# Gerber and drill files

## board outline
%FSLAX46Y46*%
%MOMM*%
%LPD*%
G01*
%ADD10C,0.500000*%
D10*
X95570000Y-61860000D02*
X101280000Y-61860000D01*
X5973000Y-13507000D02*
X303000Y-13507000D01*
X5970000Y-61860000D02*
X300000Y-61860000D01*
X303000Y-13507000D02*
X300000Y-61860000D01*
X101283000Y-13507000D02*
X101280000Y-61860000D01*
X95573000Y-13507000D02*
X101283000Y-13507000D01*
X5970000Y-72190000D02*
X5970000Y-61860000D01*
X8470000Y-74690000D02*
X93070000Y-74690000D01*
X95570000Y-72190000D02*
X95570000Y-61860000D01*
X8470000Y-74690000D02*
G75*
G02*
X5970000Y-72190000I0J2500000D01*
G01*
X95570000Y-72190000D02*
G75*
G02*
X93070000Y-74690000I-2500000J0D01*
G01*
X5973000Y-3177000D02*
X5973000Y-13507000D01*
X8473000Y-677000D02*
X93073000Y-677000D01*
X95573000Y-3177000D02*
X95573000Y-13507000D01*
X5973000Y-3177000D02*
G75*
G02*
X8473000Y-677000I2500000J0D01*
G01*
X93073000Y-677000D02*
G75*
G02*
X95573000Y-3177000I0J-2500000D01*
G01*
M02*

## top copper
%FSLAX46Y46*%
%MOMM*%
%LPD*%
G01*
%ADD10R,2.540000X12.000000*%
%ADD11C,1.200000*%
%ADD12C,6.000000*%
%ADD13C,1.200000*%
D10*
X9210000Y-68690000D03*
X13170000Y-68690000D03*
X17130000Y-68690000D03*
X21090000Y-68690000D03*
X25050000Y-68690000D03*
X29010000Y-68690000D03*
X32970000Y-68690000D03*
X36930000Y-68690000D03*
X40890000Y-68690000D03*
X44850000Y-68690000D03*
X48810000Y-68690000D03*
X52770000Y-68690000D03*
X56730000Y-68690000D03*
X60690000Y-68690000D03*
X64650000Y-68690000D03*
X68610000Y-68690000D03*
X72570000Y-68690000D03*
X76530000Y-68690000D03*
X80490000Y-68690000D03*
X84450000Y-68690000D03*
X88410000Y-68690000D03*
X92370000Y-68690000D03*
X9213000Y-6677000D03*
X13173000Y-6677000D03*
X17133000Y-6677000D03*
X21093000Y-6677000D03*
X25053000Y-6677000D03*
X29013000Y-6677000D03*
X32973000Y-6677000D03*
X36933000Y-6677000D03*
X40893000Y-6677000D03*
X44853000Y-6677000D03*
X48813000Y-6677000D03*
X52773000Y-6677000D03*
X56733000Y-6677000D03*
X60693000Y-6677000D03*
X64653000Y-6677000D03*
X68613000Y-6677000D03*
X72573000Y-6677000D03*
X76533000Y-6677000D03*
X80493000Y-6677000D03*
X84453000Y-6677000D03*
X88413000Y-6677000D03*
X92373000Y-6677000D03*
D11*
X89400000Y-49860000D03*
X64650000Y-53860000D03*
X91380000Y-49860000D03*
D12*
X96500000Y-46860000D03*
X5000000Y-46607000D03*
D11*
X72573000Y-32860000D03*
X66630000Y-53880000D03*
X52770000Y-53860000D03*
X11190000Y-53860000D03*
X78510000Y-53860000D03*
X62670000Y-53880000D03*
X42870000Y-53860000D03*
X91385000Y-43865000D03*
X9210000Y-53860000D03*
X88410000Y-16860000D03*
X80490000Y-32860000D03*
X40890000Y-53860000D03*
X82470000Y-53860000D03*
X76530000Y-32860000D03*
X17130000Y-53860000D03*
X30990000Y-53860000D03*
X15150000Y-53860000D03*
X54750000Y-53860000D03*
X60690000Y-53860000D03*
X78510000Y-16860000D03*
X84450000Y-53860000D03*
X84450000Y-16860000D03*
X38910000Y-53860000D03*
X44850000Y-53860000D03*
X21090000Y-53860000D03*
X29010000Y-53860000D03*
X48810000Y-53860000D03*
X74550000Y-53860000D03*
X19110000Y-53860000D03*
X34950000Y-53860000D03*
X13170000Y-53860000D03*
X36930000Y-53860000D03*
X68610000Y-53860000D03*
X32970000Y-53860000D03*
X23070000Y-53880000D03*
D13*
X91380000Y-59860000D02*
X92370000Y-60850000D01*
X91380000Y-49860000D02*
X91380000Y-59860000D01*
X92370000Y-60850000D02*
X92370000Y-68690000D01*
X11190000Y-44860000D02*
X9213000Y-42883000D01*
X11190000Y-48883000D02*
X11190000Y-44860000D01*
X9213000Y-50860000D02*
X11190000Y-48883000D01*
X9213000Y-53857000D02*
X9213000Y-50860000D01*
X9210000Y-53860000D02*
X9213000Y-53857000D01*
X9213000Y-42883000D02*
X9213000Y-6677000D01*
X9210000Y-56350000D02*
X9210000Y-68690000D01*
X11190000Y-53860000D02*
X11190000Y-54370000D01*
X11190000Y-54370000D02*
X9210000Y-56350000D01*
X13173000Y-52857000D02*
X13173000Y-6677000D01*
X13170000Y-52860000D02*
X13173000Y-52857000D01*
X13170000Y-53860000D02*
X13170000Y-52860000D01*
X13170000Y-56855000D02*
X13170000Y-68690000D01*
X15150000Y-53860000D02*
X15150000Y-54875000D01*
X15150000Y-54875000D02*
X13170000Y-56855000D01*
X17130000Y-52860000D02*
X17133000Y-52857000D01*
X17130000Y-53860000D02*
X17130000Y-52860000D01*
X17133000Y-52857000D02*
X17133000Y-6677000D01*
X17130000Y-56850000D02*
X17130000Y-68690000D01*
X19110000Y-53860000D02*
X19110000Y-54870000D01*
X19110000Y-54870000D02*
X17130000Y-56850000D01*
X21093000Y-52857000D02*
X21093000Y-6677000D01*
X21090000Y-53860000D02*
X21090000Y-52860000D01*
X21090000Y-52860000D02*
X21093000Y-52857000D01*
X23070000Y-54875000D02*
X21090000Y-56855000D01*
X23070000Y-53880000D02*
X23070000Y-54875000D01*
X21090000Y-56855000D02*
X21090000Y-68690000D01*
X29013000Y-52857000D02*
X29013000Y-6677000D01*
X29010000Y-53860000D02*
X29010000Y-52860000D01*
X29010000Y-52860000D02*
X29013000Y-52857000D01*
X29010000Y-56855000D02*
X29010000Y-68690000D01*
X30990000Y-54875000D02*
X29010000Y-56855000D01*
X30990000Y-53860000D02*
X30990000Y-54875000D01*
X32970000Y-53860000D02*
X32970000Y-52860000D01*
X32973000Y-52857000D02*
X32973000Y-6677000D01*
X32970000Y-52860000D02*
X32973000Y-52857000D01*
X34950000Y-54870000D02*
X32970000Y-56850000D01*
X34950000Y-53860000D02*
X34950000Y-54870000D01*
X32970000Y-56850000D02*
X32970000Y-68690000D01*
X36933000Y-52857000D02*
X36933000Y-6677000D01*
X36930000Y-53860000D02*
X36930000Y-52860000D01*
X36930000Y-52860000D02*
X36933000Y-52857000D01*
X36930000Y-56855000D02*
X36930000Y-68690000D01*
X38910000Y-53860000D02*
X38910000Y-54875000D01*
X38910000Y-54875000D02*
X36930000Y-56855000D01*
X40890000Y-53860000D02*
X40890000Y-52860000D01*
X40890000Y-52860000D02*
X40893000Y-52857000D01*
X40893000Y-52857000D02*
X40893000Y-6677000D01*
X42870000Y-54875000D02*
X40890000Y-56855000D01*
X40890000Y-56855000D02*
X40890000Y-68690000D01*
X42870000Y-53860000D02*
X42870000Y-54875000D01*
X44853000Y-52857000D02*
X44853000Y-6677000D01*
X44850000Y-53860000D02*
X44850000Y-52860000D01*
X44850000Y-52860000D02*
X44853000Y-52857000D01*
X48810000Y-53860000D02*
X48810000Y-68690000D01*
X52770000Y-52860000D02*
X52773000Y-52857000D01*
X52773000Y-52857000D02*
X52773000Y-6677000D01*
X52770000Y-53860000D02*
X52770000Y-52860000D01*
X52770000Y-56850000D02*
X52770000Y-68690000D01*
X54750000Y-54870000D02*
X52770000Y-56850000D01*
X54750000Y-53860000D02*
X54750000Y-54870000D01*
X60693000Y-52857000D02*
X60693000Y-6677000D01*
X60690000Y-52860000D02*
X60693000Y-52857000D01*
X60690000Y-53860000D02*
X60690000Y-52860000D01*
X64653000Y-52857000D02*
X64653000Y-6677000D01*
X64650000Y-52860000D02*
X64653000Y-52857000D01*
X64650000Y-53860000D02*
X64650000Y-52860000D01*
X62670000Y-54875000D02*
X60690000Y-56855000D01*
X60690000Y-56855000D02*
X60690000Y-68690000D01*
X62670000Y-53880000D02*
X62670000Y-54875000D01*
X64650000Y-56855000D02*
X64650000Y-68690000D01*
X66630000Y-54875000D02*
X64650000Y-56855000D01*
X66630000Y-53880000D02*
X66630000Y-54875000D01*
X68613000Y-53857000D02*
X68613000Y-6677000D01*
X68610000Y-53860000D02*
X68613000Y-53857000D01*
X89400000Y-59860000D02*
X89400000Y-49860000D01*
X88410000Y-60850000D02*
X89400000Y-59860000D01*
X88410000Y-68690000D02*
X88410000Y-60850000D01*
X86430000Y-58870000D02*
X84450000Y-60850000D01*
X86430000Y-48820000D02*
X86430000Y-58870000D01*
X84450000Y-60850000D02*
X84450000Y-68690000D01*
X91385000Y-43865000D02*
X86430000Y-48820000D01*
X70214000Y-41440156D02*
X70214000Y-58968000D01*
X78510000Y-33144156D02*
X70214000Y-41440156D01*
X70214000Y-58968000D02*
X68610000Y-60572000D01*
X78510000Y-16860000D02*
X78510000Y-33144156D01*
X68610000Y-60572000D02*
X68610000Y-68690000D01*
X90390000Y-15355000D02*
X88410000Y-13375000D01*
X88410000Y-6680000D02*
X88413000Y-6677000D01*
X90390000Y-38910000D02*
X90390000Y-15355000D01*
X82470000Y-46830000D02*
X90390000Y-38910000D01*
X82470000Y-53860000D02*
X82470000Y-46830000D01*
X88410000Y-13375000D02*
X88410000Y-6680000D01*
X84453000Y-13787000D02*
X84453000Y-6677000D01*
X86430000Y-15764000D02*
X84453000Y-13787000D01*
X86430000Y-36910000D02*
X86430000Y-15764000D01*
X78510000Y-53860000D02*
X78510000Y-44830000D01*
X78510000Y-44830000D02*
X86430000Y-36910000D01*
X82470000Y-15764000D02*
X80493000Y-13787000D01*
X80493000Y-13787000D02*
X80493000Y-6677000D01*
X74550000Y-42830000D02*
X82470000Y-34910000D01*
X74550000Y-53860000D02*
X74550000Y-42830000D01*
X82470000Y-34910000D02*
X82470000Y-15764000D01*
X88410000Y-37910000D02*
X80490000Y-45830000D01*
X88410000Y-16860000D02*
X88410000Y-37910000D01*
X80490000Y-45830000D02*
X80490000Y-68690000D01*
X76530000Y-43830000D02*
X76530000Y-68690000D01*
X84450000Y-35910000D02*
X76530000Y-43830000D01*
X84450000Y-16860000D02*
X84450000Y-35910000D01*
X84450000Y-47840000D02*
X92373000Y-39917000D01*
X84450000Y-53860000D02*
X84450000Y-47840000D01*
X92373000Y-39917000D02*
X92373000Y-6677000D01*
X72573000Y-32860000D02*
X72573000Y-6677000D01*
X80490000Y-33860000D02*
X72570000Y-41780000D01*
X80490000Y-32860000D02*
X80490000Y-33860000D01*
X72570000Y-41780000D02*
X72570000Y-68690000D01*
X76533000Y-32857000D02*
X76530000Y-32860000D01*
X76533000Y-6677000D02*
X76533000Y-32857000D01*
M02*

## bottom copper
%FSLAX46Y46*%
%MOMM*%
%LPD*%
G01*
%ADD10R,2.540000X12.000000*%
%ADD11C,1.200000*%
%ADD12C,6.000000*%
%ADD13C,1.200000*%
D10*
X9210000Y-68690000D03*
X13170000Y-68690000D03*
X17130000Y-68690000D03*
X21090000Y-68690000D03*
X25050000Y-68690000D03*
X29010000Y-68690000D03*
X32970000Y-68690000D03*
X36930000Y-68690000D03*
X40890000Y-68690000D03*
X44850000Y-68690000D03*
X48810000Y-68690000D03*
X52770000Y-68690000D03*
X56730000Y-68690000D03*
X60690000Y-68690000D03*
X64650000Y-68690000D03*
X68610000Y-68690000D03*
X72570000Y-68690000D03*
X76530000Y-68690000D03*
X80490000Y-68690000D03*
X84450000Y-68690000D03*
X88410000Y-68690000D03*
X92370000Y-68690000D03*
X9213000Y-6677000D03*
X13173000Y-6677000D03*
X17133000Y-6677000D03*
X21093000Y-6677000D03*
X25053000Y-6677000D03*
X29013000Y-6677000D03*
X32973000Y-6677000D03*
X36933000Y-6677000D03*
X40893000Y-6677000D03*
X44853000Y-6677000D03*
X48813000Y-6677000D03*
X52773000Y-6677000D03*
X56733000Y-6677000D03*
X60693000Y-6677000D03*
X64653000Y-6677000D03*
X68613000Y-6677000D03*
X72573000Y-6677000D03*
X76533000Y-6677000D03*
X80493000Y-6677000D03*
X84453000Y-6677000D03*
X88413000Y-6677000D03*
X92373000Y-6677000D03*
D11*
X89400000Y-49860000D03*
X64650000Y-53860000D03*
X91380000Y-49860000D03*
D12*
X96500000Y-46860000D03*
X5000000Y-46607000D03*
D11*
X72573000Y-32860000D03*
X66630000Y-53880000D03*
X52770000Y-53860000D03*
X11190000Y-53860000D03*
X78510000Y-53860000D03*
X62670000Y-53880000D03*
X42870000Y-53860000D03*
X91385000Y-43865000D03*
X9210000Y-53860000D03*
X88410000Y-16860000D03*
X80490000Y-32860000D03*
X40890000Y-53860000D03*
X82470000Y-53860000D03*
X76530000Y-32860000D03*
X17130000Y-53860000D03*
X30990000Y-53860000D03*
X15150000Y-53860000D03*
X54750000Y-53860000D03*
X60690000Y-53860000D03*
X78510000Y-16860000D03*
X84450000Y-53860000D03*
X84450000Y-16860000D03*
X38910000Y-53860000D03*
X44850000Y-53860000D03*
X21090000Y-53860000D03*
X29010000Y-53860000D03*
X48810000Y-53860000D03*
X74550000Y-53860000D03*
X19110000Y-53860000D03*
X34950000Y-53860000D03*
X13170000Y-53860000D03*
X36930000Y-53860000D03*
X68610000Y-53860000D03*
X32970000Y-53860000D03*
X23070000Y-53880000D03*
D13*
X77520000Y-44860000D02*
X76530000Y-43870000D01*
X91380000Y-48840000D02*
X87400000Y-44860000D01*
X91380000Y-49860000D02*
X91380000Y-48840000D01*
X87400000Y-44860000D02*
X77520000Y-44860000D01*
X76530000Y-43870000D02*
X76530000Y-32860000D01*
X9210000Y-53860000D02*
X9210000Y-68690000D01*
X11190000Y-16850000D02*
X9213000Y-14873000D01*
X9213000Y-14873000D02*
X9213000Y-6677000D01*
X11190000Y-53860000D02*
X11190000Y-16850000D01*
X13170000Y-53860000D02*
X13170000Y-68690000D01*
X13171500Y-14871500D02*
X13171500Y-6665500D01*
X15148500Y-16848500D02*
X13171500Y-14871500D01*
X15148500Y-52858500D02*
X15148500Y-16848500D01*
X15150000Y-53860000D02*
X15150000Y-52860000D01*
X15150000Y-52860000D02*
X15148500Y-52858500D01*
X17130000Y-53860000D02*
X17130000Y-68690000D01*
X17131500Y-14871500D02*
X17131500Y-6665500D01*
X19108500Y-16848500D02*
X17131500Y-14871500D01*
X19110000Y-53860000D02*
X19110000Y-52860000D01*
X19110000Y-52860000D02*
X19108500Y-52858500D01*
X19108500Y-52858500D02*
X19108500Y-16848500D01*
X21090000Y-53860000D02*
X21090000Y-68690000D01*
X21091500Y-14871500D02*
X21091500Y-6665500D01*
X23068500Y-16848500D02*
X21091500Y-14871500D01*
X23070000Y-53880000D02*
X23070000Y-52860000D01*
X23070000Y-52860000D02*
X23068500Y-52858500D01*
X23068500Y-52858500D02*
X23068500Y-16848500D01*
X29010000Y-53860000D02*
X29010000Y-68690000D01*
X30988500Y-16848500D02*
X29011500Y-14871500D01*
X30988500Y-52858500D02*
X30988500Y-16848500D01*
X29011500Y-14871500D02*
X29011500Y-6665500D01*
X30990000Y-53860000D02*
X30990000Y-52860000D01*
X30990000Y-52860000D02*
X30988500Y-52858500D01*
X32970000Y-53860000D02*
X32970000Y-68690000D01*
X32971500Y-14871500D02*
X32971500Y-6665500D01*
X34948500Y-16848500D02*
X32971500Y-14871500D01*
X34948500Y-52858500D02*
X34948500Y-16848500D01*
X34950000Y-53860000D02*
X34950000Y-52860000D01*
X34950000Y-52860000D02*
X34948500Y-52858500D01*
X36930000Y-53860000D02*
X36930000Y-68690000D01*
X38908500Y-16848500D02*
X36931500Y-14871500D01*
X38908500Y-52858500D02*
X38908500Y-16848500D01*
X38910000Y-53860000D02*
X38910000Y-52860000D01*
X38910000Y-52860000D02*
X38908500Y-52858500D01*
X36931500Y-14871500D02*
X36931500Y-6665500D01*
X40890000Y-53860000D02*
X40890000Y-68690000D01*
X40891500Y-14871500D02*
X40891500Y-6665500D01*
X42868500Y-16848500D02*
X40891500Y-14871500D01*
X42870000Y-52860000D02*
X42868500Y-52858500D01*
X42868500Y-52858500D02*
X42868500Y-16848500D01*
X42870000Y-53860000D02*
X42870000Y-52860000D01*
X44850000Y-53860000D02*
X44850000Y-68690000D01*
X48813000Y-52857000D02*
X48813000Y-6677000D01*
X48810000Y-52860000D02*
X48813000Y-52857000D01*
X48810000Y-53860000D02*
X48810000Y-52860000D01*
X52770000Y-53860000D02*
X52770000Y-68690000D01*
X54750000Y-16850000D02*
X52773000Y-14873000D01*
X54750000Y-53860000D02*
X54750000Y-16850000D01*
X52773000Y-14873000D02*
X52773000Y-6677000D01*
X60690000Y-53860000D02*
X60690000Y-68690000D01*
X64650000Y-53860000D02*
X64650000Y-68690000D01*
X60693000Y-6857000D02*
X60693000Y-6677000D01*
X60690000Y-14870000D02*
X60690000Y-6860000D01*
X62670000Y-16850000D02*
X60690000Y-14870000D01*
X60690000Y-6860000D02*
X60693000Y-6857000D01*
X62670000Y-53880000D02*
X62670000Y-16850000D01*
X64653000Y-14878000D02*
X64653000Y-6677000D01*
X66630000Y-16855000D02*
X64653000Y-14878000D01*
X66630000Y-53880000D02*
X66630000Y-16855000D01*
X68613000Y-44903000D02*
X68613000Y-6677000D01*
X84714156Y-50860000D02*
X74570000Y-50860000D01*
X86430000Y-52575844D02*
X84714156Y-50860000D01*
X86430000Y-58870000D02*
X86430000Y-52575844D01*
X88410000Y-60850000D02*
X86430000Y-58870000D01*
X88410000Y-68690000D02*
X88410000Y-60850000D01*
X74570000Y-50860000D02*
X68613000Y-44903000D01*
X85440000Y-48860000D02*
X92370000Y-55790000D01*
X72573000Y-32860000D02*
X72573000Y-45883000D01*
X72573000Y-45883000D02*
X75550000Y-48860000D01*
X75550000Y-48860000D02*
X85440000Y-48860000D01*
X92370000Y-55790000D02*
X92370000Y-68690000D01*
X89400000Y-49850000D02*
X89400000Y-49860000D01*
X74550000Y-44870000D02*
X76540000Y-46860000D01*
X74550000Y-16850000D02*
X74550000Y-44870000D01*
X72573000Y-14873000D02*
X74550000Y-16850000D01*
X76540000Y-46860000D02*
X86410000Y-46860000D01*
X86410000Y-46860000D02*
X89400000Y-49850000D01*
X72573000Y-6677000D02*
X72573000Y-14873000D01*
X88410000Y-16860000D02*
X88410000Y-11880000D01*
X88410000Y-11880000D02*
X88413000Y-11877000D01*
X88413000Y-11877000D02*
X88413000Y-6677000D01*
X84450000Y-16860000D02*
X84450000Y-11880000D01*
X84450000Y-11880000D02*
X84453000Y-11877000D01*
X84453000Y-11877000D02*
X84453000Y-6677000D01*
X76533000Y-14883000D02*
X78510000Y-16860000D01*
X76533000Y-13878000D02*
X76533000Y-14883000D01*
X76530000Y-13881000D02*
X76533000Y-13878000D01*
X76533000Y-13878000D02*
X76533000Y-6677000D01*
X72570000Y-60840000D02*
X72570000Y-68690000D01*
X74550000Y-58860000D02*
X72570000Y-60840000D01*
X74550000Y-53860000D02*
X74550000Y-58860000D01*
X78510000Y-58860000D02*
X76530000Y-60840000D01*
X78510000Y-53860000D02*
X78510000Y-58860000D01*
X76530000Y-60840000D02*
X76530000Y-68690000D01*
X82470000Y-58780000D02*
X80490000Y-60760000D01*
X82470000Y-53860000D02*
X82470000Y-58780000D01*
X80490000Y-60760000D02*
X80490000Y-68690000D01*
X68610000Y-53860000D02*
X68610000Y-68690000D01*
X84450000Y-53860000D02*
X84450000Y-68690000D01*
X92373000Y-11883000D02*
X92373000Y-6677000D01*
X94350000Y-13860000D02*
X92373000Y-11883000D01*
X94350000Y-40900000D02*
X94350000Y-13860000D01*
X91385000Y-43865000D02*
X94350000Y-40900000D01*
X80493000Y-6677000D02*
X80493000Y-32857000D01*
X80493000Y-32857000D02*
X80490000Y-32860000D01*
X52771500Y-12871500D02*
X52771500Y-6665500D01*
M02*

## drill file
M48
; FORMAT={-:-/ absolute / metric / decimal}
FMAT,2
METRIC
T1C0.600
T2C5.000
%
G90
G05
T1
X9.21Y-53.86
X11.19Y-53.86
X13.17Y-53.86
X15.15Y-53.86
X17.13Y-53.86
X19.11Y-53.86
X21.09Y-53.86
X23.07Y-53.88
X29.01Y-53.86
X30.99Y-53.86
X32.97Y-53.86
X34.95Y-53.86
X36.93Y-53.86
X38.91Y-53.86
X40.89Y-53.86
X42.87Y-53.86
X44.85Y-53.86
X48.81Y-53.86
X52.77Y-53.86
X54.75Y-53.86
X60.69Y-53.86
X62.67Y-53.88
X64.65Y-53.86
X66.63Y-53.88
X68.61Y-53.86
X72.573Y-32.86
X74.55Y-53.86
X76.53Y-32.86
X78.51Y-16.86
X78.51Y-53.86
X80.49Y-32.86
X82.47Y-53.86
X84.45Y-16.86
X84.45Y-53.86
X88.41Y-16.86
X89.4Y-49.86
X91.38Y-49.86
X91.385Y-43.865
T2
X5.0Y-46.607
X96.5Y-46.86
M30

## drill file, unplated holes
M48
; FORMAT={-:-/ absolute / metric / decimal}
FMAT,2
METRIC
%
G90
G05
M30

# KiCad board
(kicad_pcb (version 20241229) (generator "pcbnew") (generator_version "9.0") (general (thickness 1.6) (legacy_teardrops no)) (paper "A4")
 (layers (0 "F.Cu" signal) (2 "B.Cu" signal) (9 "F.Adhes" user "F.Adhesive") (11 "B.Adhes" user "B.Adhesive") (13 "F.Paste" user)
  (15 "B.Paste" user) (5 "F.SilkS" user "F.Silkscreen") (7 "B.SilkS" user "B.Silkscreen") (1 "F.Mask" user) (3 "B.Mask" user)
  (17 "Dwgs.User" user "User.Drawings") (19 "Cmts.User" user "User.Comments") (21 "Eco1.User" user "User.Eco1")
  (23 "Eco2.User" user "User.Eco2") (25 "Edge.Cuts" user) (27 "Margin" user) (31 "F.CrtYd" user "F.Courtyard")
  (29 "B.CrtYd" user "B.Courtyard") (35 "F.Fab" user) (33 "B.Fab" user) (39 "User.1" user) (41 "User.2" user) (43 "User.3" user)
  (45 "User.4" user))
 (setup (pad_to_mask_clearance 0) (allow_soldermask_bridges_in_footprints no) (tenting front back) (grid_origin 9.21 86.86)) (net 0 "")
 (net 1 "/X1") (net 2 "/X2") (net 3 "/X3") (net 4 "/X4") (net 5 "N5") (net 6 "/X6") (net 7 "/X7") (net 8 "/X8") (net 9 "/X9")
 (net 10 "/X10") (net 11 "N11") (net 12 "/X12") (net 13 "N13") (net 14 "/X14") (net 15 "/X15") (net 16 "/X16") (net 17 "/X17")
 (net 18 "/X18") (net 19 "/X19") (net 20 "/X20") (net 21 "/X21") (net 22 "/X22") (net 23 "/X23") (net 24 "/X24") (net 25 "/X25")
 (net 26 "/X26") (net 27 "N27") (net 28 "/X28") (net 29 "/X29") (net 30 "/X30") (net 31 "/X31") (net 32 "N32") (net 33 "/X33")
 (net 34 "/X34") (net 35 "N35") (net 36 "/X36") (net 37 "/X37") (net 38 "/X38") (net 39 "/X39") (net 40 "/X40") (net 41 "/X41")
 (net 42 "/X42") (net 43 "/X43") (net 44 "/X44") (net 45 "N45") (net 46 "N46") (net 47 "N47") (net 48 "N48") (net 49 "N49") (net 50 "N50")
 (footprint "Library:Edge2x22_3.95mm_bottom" (layer "F.Cu") (at 52.77 74.69)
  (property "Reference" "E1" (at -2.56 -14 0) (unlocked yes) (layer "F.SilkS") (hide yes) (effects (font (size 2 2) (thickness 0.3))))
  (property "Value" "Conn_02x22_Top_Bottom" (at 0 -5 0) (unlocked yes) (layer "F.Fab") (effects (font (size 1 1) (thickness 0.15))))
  (fp_line (start -46.8 -2.5) (end -46.8 -12.83) (stroke (width 0.5) (type default)) (layer "Edge.Cuts"))
  (fp_line (start -44.3 0) (end 40.3 0) (stroke (width 0.5) (type solid)) (layer "Edge.Cuts"))
  (fp_line (start 42.8 -2.5) (end 42.8 -12.83) (stroke (width 0.5) (type default)) (layer "Edge.Cuts"))
  (fp_arc (start -44.3 0) (mid -46.067767 -0.732233) (end -46.8 -2.5) (stroke (width 0.5) (type default)) (layer "Edge.Cuts"))
  (fp_arc (start 42.8 -2.5) (mid 42.067767 -0.732233) (end 40.3 0) (stroke (width 0.5) (type default)) (layer "Edge.Cuts"))
  (pad "1" connect rect (at -43.56 -6) (size 2.54 12) (layers "B.Cu" "B.Mask") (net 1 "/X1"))
  (pad "2" connect rect (at -39.6 -6) (size 2.54 12) (layers "B.Cu" "B.Mask") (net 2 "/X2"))
  (pad "3" connect rect (at -35.64 -6) (size 2.54 12) (layers "B.Cu" "B.Mask") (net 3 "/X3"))
  (pad "4" connect rect (at -31.68 -6) (size 2.54 12) (layers "B.Cu" "B.Mask") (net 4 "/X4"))
  (pad "5" connect rect (at -27.72 -6) (size 2.54 12) (layers "B.Cu" "B.Mask") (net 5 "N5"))
  (pad "6" connect rect (at -23.76 -6) (size 2.54 12) (layers "B.Cu" "B.Mask") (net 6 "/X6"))
  (pad "7" connect rect (at -19.8 -6) (size 2.54 12) (layers "B.Cu" "B.Mask") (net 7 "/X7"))
  (pad "8" connect rect (at -15.84 -6) (size 2.54 12) (layers "B.Cu" "B.Mask") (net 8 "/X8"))
  (pad "9" connect rect (at -11.88 -6) (size 2.54 12) (layers "B.Cu" "B.Mask") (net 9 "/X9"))
  (pad "10" connect rect (at -7.92 -6) (size 2.54 12) (layers "B.Cu" "B.Mask") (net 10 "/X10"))
  (pad "11" connect rect (at -3.96 -6) (size 2.54 12) (layers "B.Cu" "B.Mask") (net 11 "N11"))
  (pad "12" connect rect (at 0 -6) (size 2.54 12) (layers "B.Cu" "B.Mask") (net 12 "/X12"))
  (pad "13" connect rect (at 3.96 -6) (size 2.54 12) (layers "B.Cu" "B.Mask") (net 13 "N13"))
  (pad "14" connect rect (at 7.92 -6) (size 2.54 12) (layers "B.Cu" "B.Mask") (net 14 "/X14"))
  (pad "15" connect rect (at 11.88 -6) (size 2.54 12) (layers "B.Cu" "B.Mask") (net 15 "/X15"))
  (pad "16" connect rect (at 15.84 -6) (size 2.54 12) (layers "B.Cu" "B.Mask") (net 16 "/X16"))
  (pad "17" connect rect (at 19.8 -6) (size 2.54 12) (layers "B.Cu" "B.Mask") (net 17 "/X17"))
  (pad "18" connect rect (at 23.76 -6) (size 2.54 12) (layers "B.Cu" "B.Mask") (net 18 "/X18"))
  (pad "19" connect rect (at 27.72 -6) (size 2.54 12) (layers "B.Cu" "B.Mask") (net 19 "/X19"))
  (pad "20" connect rect (at 31.68 -6) (size 2.54 12) (layers "B.Cu" "B.Mask") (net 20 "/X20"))
  (pad "21" connect rect (at 35.64 -6) (size 2.54 12) (layers "B.Cu" "B.Mask") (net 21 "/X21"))
  (pad "22" connect rect (at 39.6 -6) (size 2.54 12) (layers "B.Cu" "B.Mask") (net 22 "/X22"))
  (pad "23" connect rect (at -43.56 -6) (size 2.54 12) (layers "F.Cu" "F.Mask") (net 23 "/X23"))
  (pad "24" connect rect (at -39.6 -6) (size 2.54 12) (layers "F.Cu" "F.Mask") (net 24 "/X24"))
  (pad "25" connect rect (at -35.64 -6) (size 2.54 12) (layers "F.Cu" "F.Mask") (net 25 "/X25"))
  (pad "26" connect rect (at -31.68 -6) (size 2.54 12) (layers "F.Cu" "F.Mask") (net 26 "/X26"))
  (pad "27" connect rect (at -27.72 -6) (size 2.54 12) (layers "F.Cu" "F.Mask") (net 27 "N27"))
  (pad "28" connect rect (at -23.76 -6) (size 2.54 12) (layers "F.Cu" "F.Mask") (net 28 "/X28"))
  (pad "29" connect rect (at -19.8 -6) (size 2.54 12) (layers "F.Cu" "F.Mask") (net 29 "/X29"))
  (pad "30" connect rect (at -15.84 -6) (size 2.54 12) (layers "F.Cu" "F.Mask") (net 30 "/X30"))
  (pad "31" connect rect (at -11.88 -6) (size 2.54 12) (layers "F.Cu" "F.Mask") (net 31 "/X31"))
  (pad "32" connect rect (at -7.92 -6) (size 2.54 12) (layers "F.Cu" "F.Mask") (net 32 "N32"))
  (pad "33" connect rect (at -3.96 -6) (size 2.54 12) (layers "F.Cu" "F.Mask") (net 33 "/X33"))
  (pad "34" connect rect (at 0 -6) (size 2.54 12) (layers "F.Cu" "F.Mask") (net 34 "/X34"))
  (pad "35" connect rect (at 3.96 -6) (size 2.54 12) (layers "F.Cu" "F.Mask") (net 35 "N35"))
  (pad "36" connect rect (at 7.92 -6) (size 2.54 12) (layers "F.Cu" "F.Mask") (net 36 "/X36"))
  (pad "37" connect rect (at 11.88 -6) (size 2.54 12) (layers "F.Cu" "F.Mask") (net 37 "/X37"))
  (pad "38" connect rect (at 15.84 -6) (size 2.54 12) (layers "F.Cu" "F.Mask") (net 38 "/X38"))
  (pad "39" connect rect (at 19.8 -6) (size 2.54 12) (layers "F.Cu" "F.Mask") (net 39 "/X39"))
  (pad "40" connect rect (at 23.76 -6) (size 2.54 12) (layers "F.Cu" "F.Mask") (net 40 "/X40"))
  (pad "41" connect rect (at 27.72 -6) (size 2.54 12) (layers "F.Cu" "F.Mask") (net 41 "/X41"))
  (pad "42" connect rect (at 31.68 -6) (size 2.54 12) (layers "F.Cu" "F.Mask") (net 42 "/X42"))
  (pad "43" connect rect (at 35.64 -6) (size 2.54 12) (layers "F.Cu" "F.Mask") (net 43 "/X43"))
  (pad "44" connect rect (at 39.6 -6) (size 2.54 12) (layers "F.Cu" "F.Mask") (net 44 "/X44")))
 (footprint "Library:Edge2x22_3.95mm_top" (layer "F.Cu") (at 52.773 12.677)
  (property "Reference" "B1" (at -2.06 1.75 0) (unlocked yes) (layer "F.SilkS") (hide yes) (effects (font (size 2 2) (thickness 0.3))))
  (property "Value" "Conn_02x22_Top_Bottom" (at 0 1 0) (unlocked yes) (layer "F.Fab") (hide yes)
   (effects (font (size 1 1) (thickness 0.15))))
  (fp_line (start -46.8 -9.5) (end -46.8 0.83) (stroke (width 0.5) (type default)) (layer "Edge.Cuts"))
  (fp_line (start -44.3 -12) (end 40.3 -12) (stroke (width 0.5) (type solid)) (layer "Edge.Cuts"))
  (fp_line (start 42.8 -9.5) (end 42.8 0.83) (stroke (width 0.5) (type default)) (layer "Edge.Cuts"))
  (fp_arc (start -46.8 -9.5) (mid -46.067767 -11.267767) (end -44.3 -12) (stroke (width 0.5) (type default)) (layer "Edge.Cuts"))
  (fp_arc (start 40.3 -12) (mid 42.067767 -11.267767) (end 42.8 -9.5) (stroke (width 0.5) (type default)) (layer "Edge.Cuts"))
  (pad "1" connect rect (at -43.56 -6) (size 2.54 12) (layers "F.Cu" "F.Mask") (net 1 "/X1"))
  (pad "2" connect rect (at -39.6 -6) (size 2.54 12) (layers "F.Cu" "F.Mask") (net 2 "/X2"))
  (pad "3" connect rect (at -35.64 -6) (size 2.54 12) (layers "F.Cu" "F.Mask") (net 3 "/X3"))
  (pad "4" connect rect (at -31.68 -6) (size 2.54 12) (layers "F.Cu" "F.Mask") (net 4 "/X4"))
  (pad "5" connect rect (at -27.72 -6) (size 2.54 12) (layers "F.Cu" "F.Mask") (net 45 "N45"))
  (pad "6" connect rect (at -23.76 -6) (size 2.54 12) (layers "F.Cu" "F.Mask") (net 6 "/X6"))
  (pad "7" connect rect (at -19.8 -6) (size 2.54 12) (layers "F.Cu" "F.Mask") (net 7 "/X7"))
  (pad "8" connect rect (at -15.84 -6) (size 2.54 12) (layers "F.Cu" "F.Mask") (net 8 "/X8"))
  (pad "9" connect rect (at -11.88 -6) (size 2.54 12) (layers "F.Cu" "F.Mask") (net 9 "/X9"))
  (pad "10" connect rect (at -7.92 -6) (size 2.54 12) (layers "F.Cu" "F.Mask") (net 10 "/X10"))
  (pad "11" connect rect (at -3.96 -6) (size 2.54 12) (layers "F.Cu" "F.Mask") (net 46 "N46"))
  (pad "12" connect rect (at 0 -6) (size 2.54 12) (layers "F.Cu" "F.Mask") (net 12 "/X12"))
  (pad "13" connect rect (at 3.96 -6) (size 2.54 12) (layers "F.Cu" "F.Mask") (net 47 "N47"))
  (pad "14" connect rect (at 7.92 -6) (size 2.54 12) (layers "F.Cu" "F.Mask") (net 14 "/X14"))
  (pad "15" connect rect (at 11.88 -6) (size 2.54 12) (layers "F.Cu" "F.Mask") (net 15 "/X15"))
  (pad "16" connect rect (at 15.84 -6) (size 2.54 12) (layers "F.Cu" "F.Mask") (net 16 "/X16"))
  (pad "17" connect rect (at 19.8 -6) (size 2.54 12) (layers "F.Cu" "F.Mask") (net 22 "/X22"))
  (pad "18" connect rect (at 23.76 -6) (size 2.54 12) (layers "F.Cu" "F.Mask") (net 44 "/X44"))
  (pad "19" connect rect (at 27.72 -6) (size 2.54 12) (layers "F.Cu" "F.Mask") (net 17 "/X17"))
  (pad "20" connect rect (at 31.68 -6) (size 2.54 12) (layers "F.Cu" "F.Mask") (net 18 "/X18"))
  (pad "21" connect rect (at 35.64 -6) (size 2.54 12) (layers "F.Cu" "F.Mask") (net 19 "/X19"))
  (pad "22" connect rect (at 39.6 -6) (size 2.54 12) (layers "F.Cu" "F.Mask") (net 20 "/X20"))
  (pad "23" connect rect (at -43.56 -6) (size 2.54 12) (layers "B.Cu" "B.Mask") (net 23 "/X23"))
  (pad "24" connect rect (at -39.6 -6) (size 2.54 12) (layers "B.Cu" "B.Mask") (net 24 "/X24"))
  (pad "25" connect rect (at -35.64 -6) (size 2.54 12) (layers "B.Cu" "B.Mask") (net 25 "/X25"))
  (pad "26" connect rect (at -31.68 -6) (size 2.54 12) (layers "B.Cu" "B.Mask") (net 26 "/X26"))
  (pad "27" connect rect (at -27.72 -6) (size 2.54 12) (layers "B.Cu" "B.Mask") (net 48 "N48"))
  (pad "28" connect rect (at -23.76 -6) (size 2.54 12) (layers "B.Cu" "B.Mask") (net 28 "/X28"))
  (pad "29" connect rect (at -19.8 -6) (size 2.54 12) (layers "B.Cu" "B.Mask") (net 29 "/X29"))
  (pad "30" connect rect (at -15.84 -6) (size 2.54 12) (layers "B.Cu" "B.Mask") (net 30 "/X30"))
  (pad "31" connect rect (at -11.88 -6) (size 2.54 12) (layers "B.Cu" "B.Mask") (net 31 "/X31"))
  (pad "32" connect rect (at -7.92 -6) (size 2.54 12) (layers "B.Cu" "B.Mask") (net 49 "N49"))
  (pad "33" connect rect (at -3.96 -6) (size 2.54 12) (layers "B.Cu" "B.Mask") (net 33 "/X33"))
  (pad "34" connect rect (at 0 -6) (size 2.54 12) (layers "B.Cu" "B.Mask") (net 34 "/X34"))
  (pad "35" connect rect (at 3.96 -6) (size 2.54 12) (layers "B.Cu" "B.Mask") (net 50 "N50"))
  (pad "36" connect rect (at 7.92 -6) (size 2.54 12) (layers "B.Cu" "B.Mask") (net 36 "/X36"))
  (pad "37" connect rect (at 11.88 -6) (size 2.54 12) (layers "B.Cu" "B.Mask") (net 37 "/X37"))
  (pad "38" connect rect (at 15.84 -6) (size 2.54 12) (layers "B.Cu" "B.Mask") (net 21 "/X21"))
  (pad "39" connect rect (at 19.8 -6) (size 2.54 12) (layers "B.Cu" "B.Mask") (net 43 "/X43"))
  (pad "40" connect rect (at 23.76 -6) (size 2.54 12) (layers "B.Cu" "B.Mask") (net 38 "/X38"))
  (pad "41" connect rect (at 27.72 -6) (size 2.54 12) (layers "B.Cu" "B.Mask") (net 39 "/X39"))
  (pad "42" connect rect (at 31.68 -6) (size 2.54 12) (layers "B.Cu" "B.Mask") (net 40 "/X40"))
  (pad "43" connect rect (at 35.64 -6) (size 2.54 12) (layers "B.Cu" "B.Mask") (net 41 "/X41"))
  (pad "44" connect rect (at 39.6 -6) (size 2.54 12) (layers "B.Cu" "B.Mask") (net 42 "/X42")))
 (gr_line (start 95.573 13.507) (end 101.283 13.507) (stroke (width 0.5) (type default)) (layer "Edge.Cuts"))
 (gr_line (start 95.57 61.86) (end 101.28 61.86) (stroke (width 0.5) (type default)) (layer "Edge.Cuts"))
 (gr_line (start 5.973 13.507) (end 0.303 13.507) (stroke (width 0.5) (type default)) (layer "Edge.Cuts"))
 (gr_line (start 5.97 61.86) (end 0.3 61.86) (stroke (width 0.5) (type default)) (layer "Edge.Cuts"))
 (gr_line (start 0.303 13.507) (end 0.3 61.86) (stroke (width 0.5) (type default)) (layer "Edge.Cuts"))
 (gr_line (start 101.283 13.507) (end 101.28 61.86) (stroke (width 0.5) (type default)) (layer "Edge.Cuts"))
 (via (at 5 46.607) (size 6) (drill 5) (layers "F.Cu" "B.Cu") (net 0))
 (via (at 96.5 46.86) (size 6) (drill 5) (layers "F.Cu" "B.Cu") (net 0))
 (segment (start 72.573 32.86) (end 72.573 6.677) (width 1.2) (layer "F.Cu") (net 22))
 (via (at 72.573 32.86) (size 1.2) (drill 0.6) (layers "F.Cu" "B.Cu") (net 22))
 (segment (start 92.37 55.79) (end 92.37 68.69) (width 1.2) (layer "B.Cu") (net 22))
 (segment (start 72.573 32.86) (end 72.573 45.883) (width 1.2) (layer "B.Cu") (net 22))
 (segment (start 75.55 48.86) (end 85.44 48.86) (width 1.2) (layer "B.Cu") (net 22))
 (segment (start 85.44 48.86) (end 92.37 55.79) (width 1.2) (layer "B.Cu") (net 22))
 (segment (start 72.573 45.883) (end 75.55 48.86) (width 1.2) (layer "B.Cu") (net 22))
 (segment (start 88.41 68.69) (end 88.41 60.85) (width 1.2) (layer "B.Cu") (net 21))
 (segment (start 74.57 50.86) (end 68.613 44.903) (width 1.2) (layer "B.Cu") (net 21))
 (segment (start 68.613 44.903) (end 68.613 6.677) (width 1.2) (layer "B.Cu") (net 21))
 (segment (start 84.714156 50.86) (end 74.57 50.86) (width 1.2) (layer "B.Cu") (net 21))
 (segment (start 86.43 58.87) (end 86.43 52.575844) (width 1.2) (layer "B.Cu") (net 21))
 (segment (start 86.43 52.575844) (end 84.714156 50.86) (width 1.2) (layer "B.Cu") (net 21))
 (segment (start 88.41 60.85) (end 86.43 58.87) (width 1.2) (layer "B.Cu") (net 21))
 (segment (start 66.63 54.875) (end 64.65 56.855) (width 1.2) (layer "F.Cu") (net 37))
 (segment (start 64.65 56.855) (end 64.65 68.69) (width 1.2) (layer "F.Cu") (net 37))
 (segment (start 66.63 53.88) (end 66.63 54.875) (width 1.2) (layer "F.Cu") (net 37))
 (via (at 66.63 53.88) (size 1.2) (drill 0.6) (layers "F.Cu" "B.Cu") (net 37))
 (segment (start 66.63 16.855) (end 64.653 14.878) (width 1.2) (layer "B.Cu") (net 37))
 (segment (start 64.653 14.878) (end 64.653 6.677) (width 1.2) (layer "B.Cu") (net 37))
 (segment (start 66.63 53.88) (end 66.63 16.855) (width 1.2) (layer "B.Cu") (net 37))
 (segment (start 52.77 53.86) (end 52.77 52.86) (width 1.2) (layer "F.Cu") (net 12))
 (segment (start 52.773 52.857) (end 52.773 6.677) (width 1.2) (layer "F.Cu") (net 12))
 (segment (start 52.77 52.86) (end 52.773 52.857) (width 1.2) (layer "F.Cu") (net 12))
 (via (at 52.77 53.86) (size 1.2) (drill 0.6) (layers "F.Cu" "B.Cu") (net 12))
 (segment (start 52.77 53.86) (end 52.77 68.69) (width 1.2) (layer "B.Cu") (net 12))
 (segment (start 9.21 56.35) (end 9.21 68.69) (width 1.2) (layer "F.Cu") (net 23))
 (segment (start 11.19 53.86) (end 11.19 54.37) (width 1.2) (layer "F.Cu") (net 23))
 (segment (start 11.19 54.37) (end 9.21 56.35) (width 1.2) (layer "F.Cu") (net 23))
 (via (at 11.19 53.86) (size 1.2) (drill 0.6) (layers "F.Cu" "B.Cu") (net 23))
 (segment (start 11.19 16.85) (end 9.213 14.873) (width 1.2) (layer "B.Cu") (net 23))
 (segment (start 9.213 14.873) (end 9.213 6.677) (width 1.2) (layer "B.Cu") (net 23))
 (segment (start 11.19 53.86) (end 11.19 16.85) (width 1.2) (layer "B.Cu") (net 23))
 (segment (start 86.43 36.91) (end 86.43 15.764) (width 1.2) (layer "F.Cu") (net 18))
 (segment (start 86.43 15.764) (end 84.453 13.787) (width 1.2) (layer "F.Cu") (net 18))
 (segment (start 84.453 13.787) (end 84.453 6.677) (width 1.2) (layer "F.Cu") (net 18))
 (segment (start 78.51 44.83) (end 86.43 36.91) (width 1.2) (layer "F.Cu") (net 18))
 (segment (start 78.51 53.86) (end 78.51 44.83) (width 1.2) (layer "F.Cu") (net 18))
 (via (at 78.51 53.86) (size 1.2) (drill 0.6) (layers "F.Cu" "B.Cu") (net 18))
 (segment (start 76.53 60.84) (end 76.53 68.69) (width 1.2) (layer "B.Cu") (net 18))
 (segment (start 78.51 58.86) (end 76.53 60.84) (width 1.2) (layer "B.Cu") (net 18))
 (segment (start 78.51 53.86) (end 78.51 58.86) (width 1.2) (layer "B.Cu") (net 18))
 (segment (start 62.67 53.88) (end 62.67 54.875) (width 1.2) (layer "F.Cu") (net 36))
 (segment (start 62.67 54.875) (end 60.69 56.855) (width 1.2) (layer "F.Cu") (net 36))
 (segment (start 60.69 56.855) (end 60.69 68.69) (width 1.2) (layer "F.Cu") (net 36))
 (via (at 62.67 53.88) (size 1.2) (drill 0.6) (layers "F.Cu" "B.Cu") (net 36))
 (segment (start 60.69 14.87) (end 60.69 6.86) (width 1.2) (layer "B.Cu") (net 36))
 (segment (start 60.693 6.857) (end 60.693 6.677) (width 1.2) (layer "B.Cu") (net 36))
 (segment (start 62.67 16.85) (end 60.69 14.87) (width 1.2) (layer "B.Cu") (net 36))
 (segment (start 62.67 53.88) (end 62.67 16.85) (width 1.2) (layer "B.Cu") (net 36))
 (segment (start 60.69 6.86) (end 60.693 6.857) (width 1.2) (layer "B.Cu") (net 36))
 (segment (start 40.89 56.855) (end 40.89 68.69) (width 1.2) (layer "F.Cu") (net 31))
 (segment (start 42.87 53.86) (end 42.87 54.875) (width 1.2) (layer "F.Cu") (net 31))
 (segment (start 42.87 54.875) (end 40.89 56.855) (width 1.2) (layer "F.Cu") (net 31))
 (via (at 42.87 53.86) (size 1.2) (drill 0.6) (layers "F.Cu" "B.Cu") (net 31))
 (segment (start 42.87 53.86) (end 42.87 52.86) (width 1.2) (layer "B.Cu") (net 31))
 (segment (start 42.8685 16.8485) (end 40.8915 14.8715) (width 1.2) (layer "B.Cu") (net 31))
 (segment (start 42.8685 52.8585) (end 42.8685 16.8485) (width 1.2) (layer "B.Cu") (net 31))
 (segment (start 42.87 52.86) (end 42.8685 52.8585) (width 1.2) (layer "B.Cu") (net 31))
 (segment (start 40.8915 14.8715) (end 40.8915 6.6655) (width 1.2) (layer "B.Cu") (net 31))
 (segment (start 86.43 58.87) (end 84.45 60.85) (width 1.2) (layer "F.Cu") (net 42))
 (segment (start 91.385 43.865) (end 86.43 48.82) (width 1.2) (layer "F.Cu") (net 42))
 (segment (start 86.43 48.82) (end 86.43 58.87) (width 1.2) (layer "F.Cu") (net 42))
 (segment (start 84.45 60.85) (end 84.45 68.69) (width 1.2) (layer "F.Cu") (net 42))
 (via (at 91.385 43.865) (size 1.2) (drill 0.6) (layers "F.Cu" "B.Cu") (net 42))
 (segment (start 94.35 13.86) (end 92.373 11.883) (width 1.2) (layer "B.Cu") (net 42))
 (segment (start 92.373 11.883) (end 92.373 6.677) (width 1.2) (layer "B.Cu") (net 42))
 (segment (start 91.385 43.865) (end 94.35 40.9) (width 1.2) (layer "B.Cu") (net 42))
 (segment (start 94.35 40.9) (end 94.35 13.86) (width 1.2) (layer "B.Cu") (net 42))
 (segment (start 11.19 44.86) (end 9.213 42.883) (width 1.2) (layer "F.Cu") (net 1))
 (segment (start 9.213 50.86) (end 11.19 48.883) (width 1.2) (layer "F.Cu") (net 1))
 (segment (start 11.19 48.883) (end 11.19 44.86) (width 1.2) (layer "F.Cu") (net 1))
 (segment (start 9.213 53.857) (end 9.213 50.86) (width 1.2) (layer "F.Cu") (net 1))
 (segment (start 9.21 53.86) (end 9.213 53.857) (width 1.2) (layer "F.Cu") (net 1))
 (segment (start 9.213 42.883) (end 9.213 6.677) (width 1.2) (layer "F.Cu") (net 1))
 (via (at 9.21 53.86) (size 1.2) (drill 0.6) (layers "F.Cu" "B.Cu") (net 1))
 (segment (start 9.21 53.86) (end 9.21 68.69) (width 1.2) (layer "B.Cu") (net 1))
 (segment (start 88.41 37.91) (end 80.49 45.83) (width 1.2) (layer "F.Cu") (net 41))
 (segment (start 88.41 16.86) (end 88.41 37.91) (width 1.2) (layer "F.Cu") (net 41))
 (segment (start 80.49 45.83) (end 80.49 68.69) (width 1.2) (layer "F.Cu") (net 41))
 (via (at 88.41 16.86) (size 1.2) (drill 0.6) (layers "F.Cu" "B.Cu") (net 41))
 (segment (start 88.41 16.86) (end 88.41 11.88) (width 1.2) (layer "B.Cu") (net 41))
 (segment (start 88.41 11.88) (end 88.413 11.877) (width 1.2) (layer "B.Cu") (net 41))
 (segment (start 88.413 11.877) (end 88.413 6.677) (width 1.2) (layer "B.Cu") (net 41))
 (segment (start 80.49 33.86) (end 72.57 41.78) (width 1.2) (layer "F.Cu") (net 39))
 (segment (start 80.49 32.86) (end 80.49 33.86) (width 1.2) (layer "F.Cu") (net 39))
 (segment (start 72.57 41.78) (end 72.57 68.69) (width 1.2) (layer "F.Cu") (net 39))
 (via (at 80.49 32.86) (size 1.2) (drill 0.6) (layers "F.Cu" "B.Cu") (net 39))
 (segment (start 80.493 6.677) (end 80.493 32.857) (width 1.2) (layer "B.Cu") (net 39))
 (segment (start 80.493 32.857) (end 80.49 32.86) (width 1.2) (layer "B.Cu") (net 39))
 (segment (start 40.89 53.86) (end 40.89 52.86) (width 1.2) (layer "F.Cu") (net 9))
 (segment (start 40.893 52.857) (end 40.893 6.677) (width 1.2) (layer "F.Cu") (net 9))
 (segment (start 40.89 52.86) (end 40.893 52.857) (width 1.2) (layer "F.Cu") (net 9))
 (via (at 40.89 53.86) (size 1.2) (drill 0.6) (layers "F.Cu" "B.Cu") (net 9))
 (segment (start 40.89 53.86) (end 40.89 68.69) (width 1.2) (layer "B.Cu") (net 9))
 (segment (start 90.39 38.91) (end 90.39 15.355) (width 1.2) (layer "F.Cu") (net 19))
 (segment (start 88.41 13.375) (end 88.41 6.68) (width 1.2) (layer "F.Cu") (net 19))
 (segment (start 90.39 15.355) (end 88.41 13.375) (width 1.2) (layer "F.Cu") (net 19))
 (segment (start 88.41 6.68) (end 88.413 6.677) (width 1.2) (layer "F.Cu") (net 19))
 (segment (start 82.47 53.86) (end 82.47 46.83) (width 1.2) (layer "F.Cu") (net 19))
 (segment (start 82.47 46.83) (end 90.39 38.91) (width 1.2) (layer "F.Cu") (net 19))
 (via (at 82.47 53.86) (size 1.2) (drill 0.6) (layers "F.Cu" "B.Cu") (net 19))
 (segment (start 82.47 58.78) (end 80.49 60.76) (width 1.2) (layer "B.Cu") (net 19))
 (segment (start 82.47 53.86) (end 82.47 58.78) (width 1.2) (layer "B.Cu") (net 19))
 (segment (start 80.49 60.76) (end 80.49 68.69) (width 1.2) (layer "B.Cu") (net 19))
 (segment (start 88.41 60.85) (end 89.4 59.86) (width 1.2) (layer "F.Cu") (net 43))
 (segment (start 89.4 59.86) (end 89.4 49.86) (width 1.2) (layer "F.Cu") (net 43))
 (segment (start 88.41 68.69) (end 88.41 60.85) (width 1.2) (layer "F.Cu") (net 43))
 (via (at 89.4 49.86) (size 1.2) (drill 0.6) (layers "F.Cu" "B.Cu") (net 43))
 (segment (start 76.54 46.86) (end 86.41 46.86) (width 1.2) (layer "B.Cu") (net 43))
 (segment (start 74.55 16.85) (end 74.55 44.87) (width 1.2) (layer "B.Cu") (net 43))
 (segment (start 86.41 46.86) (end 89.4 49.85) (width 1.2) (layer "B.Cu") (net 43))
 (segment (start 72.573 14.873) (end 74.55 16.85) (width 1.2) (layer "B.Cu") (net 43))
 (segment (start 72.573 6.677) (end 72.573 14.873) (width 1.2) (layer "B.Cu") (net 43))
 (segment (start 74.55 44.87) (end 76.54 46.86) (width 1.2) (layer "B.Cu") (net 43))
 (segment (start 89.4 49.85) (end 89.4 49.86) (width 1.2) (layer "B.Cu") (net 43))
 (segment (start 92.37 60.85) (end 92.37 68.69) (width 1.2) (layer "F.Cu") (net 44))
 (segment (start 76.533 32.857) (end 76.53 32.86) (width 1.2) (layer "F.Cu") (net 44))
 (segment (start 91.38 59.86) (end 92.37 60.85) (width 1.2) (layer "F.Cu") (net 44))
 (segment (start 76.533 6.677) (end 76.533 32.857) (width 1.2) (layer "F.Cu") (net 44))
 (segment (start 91.38 49.86) (end 91.38 59.86) (width 1.2) (layer "F.Cu") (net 44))
 (via (at 91.38 49.86) (size 1.2) (drill 0.6) (layers "F.Cu" "B.Cu") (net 44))
 (via (at 76.53 32.86) (size 1.2) (drill 0.6) (layers "F.Cu" "B.Cu") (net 44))
 (segment (start 91.38 49.86) (end 91.38 48.84) (width 1.2) (layer "B.Cu") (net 44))
 (segment (start 87.4 44.86) (end 77.52 44.86) (width 1.2) (layer "B.Cu") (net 44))
 (segment (start 91.38 48.84) (end 87.4 44.86) (width 1.2) (layer "B.Cu") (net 44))
 (segment (start 76.53 43.87) (end 76.53 32.86) (width 1.2) (layer "B.Cu") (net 44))
 (segment (start 77.52 44.86) (end 76.53 43.87) (width 1.2) (layer "B.Cu") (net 44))
 (segment (start 17.13 53.86) (end 17.13 52.86) (width 1.2) (layer "F.Cu") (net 3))
 (segment (start 17.13 52.86) (end 17.133 52.857) (width 1.2) (layer "F.Cu") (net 3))
 (segment (start 17.133 52.857) (end 17.133 6.677) (width 1.2) (layer "F.Cu") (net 3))
 (via (at 17.13 53.86) (size 1.2) (drill 0.6) (layers "F.Cu" "B.Cu") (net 3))
 (segment (start 17.13 53.86) (end 17.13 68.69) (width 1.2) (layer "B.Cu") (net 3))
 (segment (start 29.01 56.855) (end 29.01 68.69) (width 1.2) (layer "F.Cu") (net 28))
 (segment (start 30.99 53.86) (end 30.99 54.875) (width 1.2) (layer "F.Cu") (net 28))
 (segment (start 30.99 54.875) (end 29.01 56.855) (width 1.2) (layer "F.Cu") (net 28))
 (via (at 30.99 53.86) (size 1.2) (drill 0.6) (layers "F.Cu" "B.Cu") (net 28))
 (segment (start 30.99 52.86) (end 30.9885 52.8585) (width 1.2) (layer "B.Cu") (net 28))
 (segment (start 30.99 53.86) (end 30.99 52.86) (width 1.2) (layer "B.Cu") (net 28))
 (segment (start 30.9885 16.8485) (end 29.0115 14.8715) (width 1.2) (layer "B.Cu") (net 28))
 (segment (start 29.0115 14.8715) (end 29.0115 6.6655) (width 1.2) (layer "B.Cu") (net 28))
 (segment (start 30.9885 52.8585) (end 30.9885 16.8485) (width 1.2) (layer "B.Cu") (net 28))
 (segment (start 15.15 53.86) (end 15.15 54.875) (width 1.2) (layer "F.Cu") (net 24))
 (segment (start 15.15 54.875) (end 13.17 56.855) (width 1.2) (layer "F.Cu") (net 24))
 (segment (start 13.17 56.855) (end 13.17 68.69) (width 1.2) (layer "F.Cu") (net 24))
 (via (at 15.15 53.86) (size 1.2) (drill 0.6) (layers "F.Cu" "B.Cu") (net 24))
 (segment (start 15.15 52.86) (end 15.1485 52.8585) (width 1.2) (layer "B.Cu") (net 24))
 (segment (start 15.1485 16.8485) (end 13.1715 14.8715) (width 1.2) (layer "B.Cu") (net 24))
 (segment (start 15.15 53.86) (end 15.15 52.86) (width 1.2) (layer "B.Cu") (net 24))
 (segment (start 13.1715 14.8715) (end 13.1715 6.6655) (width 1.2) (layer "B.Cu") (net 24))
 (segment (start 15.1485 52.8585) (end 15.1485 16.8485) (width 1.2) (layer "B.Cu") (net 24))
 (segment (start 54.75 54.87) (end 52.77 56.85) (width 1.2) (layer "F.Cu") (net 34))
 (segment (start 52.77 56.85) (end 52.77 68.69) (width 1.2) (layer "F.Cu") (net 34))
 (segment (start 54.75 53.86) (end 54.75 54.87) (width 1.2) (layer "F.Cu") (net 34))
 (via (at 54.75 53.86) (size 1.2) (drill 0.6) (layers "F.Cu" "B.Cu") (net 34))
 (segment (start 52.7715 12.8715) (end 52.7715 6.6655) (width 1.2) (layer "B.Cu") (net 34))
 (segment (start 54.75 53.86) (end 54.75 16.85) (width 1.2) (layer "B.Cu") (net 34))
 (segment (start 54.75 16.85) (end 52.773 14.873) (width 1.2) (layer "B.Cu") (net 34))
 (segment (start 52.773 14.873) (end 52.773 6.677) (width 1.2) (layer "B.Cu") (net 34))
 (segment (start 60.69 52.86) (end 60.693 52.857) (width 1.2) (layer "F.Cu") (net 14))
 (segment (start 60.693 52.857) (end 60.693 6.677) (width 1.2) (layer "F.Cu") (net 14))
 (segment (start 60.69 53.86) (end 60.69 52.86) (width 1.2) (layer "F.Cu") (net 14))
 (via (at 60.69 53.86) (size 1.2) (drill 0.6) (layers "F.Cu" "B.Cu") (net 14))
 (segment (start 60.69 53.86) (end 60.69 68.69) (width 1.2) (layer "B.Cu") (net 14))
 (segment (start 78.51 33.144156) (end 70.214 41.440156) (width 1.2) (layer "F.Cu") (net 38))
 (segment (start 68.61 60.572) (end 68.61 68.69) (width 1.2) (layer "F.Cu") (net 38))
 (segment (start 70.214 58.968) (end 68.61 60.572) (width 1.2) (layer "F.Cu") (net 38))
 (segment (start 78.51 16.86) (end 78.51 33.144156) (width 1.2) (layer "F.Cu") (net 38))
 (segment (start 70.214 41.440156) (end 70.214 58.968) (width 1.2) (layer "F.Cu") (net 38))
 (via (at 78.51 16.86) (size 1.2) (drill 0.6) (layers "F.Cu" "B.Cu") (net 38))
 (segment (start 76.533 13.878) (end 76.533 6.677) (width 1.2) (layer "B.Cu") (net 38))
 (segment (start 76.533 14.883) (end 78.51 16.86) (width 1.2) (layer "B.Cu") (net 38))
 (segment (start 76.533 13.878) (end 76.533 14.883) (width 1.2) (layer "B.Cu") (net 38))
 (segment (start 76.53 13.881) (end 76.533 13.878) (width 1.2) (layer "B.Cu") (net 38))
 (segment (start 84.45 47.84) (end 92.373 39.917) (width 1.2) (layer "F.Cu") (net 20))
 (segment (start 92.373 39.917) (end 92.373 6.677) (width 1.2) (layer "F.Cu") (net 20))
 (segment (start 84.45 53.86) (end 84.45 47.84) (width 1.2) (layer "F.Cu") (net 20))
 (via (at 84.45 53.86) (size 1.2) (drill 0.6) (layers "F.Cu" "B.Cu") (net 20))
 (segment (start 84.45 53.86) (end 84.45 68.69) (width 1.2) (layer "B.Cu") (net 20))
 (segment (start 84.45 16.86) (end 84.45 35.91) (width 1.2) (layer "F.Cu") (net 40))
 (segment (start 76.53 43.83) (end 76.53 68.69) (width 1.2) (layer "F.Cu") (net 40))
 (segment (start 84.45 35.91) (end 76.53 43.83) (width 1.2) (layer "F.Cu") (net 40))
 (via (at 84.45 16.86) (size 1.2) (drill 0.6) (layers "F.Cu" "B.Cu") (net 40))
 (segment (start 84.45 16.86) (end 84.45 11.88) (width 1.2) (layer "B.Cu") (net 40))
 (segment (start 84.45 11.88) (end 84.453 11.877) (width 1.2) (layer "B.Cu") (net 40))
 (segment (start 84.453 11.877) (end 84.453 6.677) (width 1.2) (layer "B.Cu") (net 40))
 (segment (start 38.91 53.86) (end 38.91 54.875) (width 1.2) (layer "F.Cu") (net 30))
 (segment (start 38.91 54.875) (end 36.93 56.855) (width 1.2) (layer "F.Cu") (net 30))
 (segment (start 36.93 56.855) (end 36.93 68.69) (width 1.2) (layer "F.Cu") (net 30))
 (via (at 38.91 53.86) (size 1.2) (drill 0.6) (layers "F.Cu" "B.Cu") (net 30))
 (segment (start 38.9085 16.8485) (end 36.9315 14.8715) (width 1.2) (layer "B.Cu") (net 30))
 (segment (start 36.9315 14.8715) (end 36.9315 6.6655) (width 1.2) (layer "B.Cu") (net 30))
 (segment (start 38.91 53.86) (end 38.91 52.86) (width 1.2) (layer "B.Cu") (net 30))
 (segment (start 38.9085 52.8585) (end 38.9085 16.8485) (width 1.2) (layer "B.Cu") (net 30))
 (segment (start 38.91 52.86) (end 38.9085 52.8585) (width 1.2) (layer "B.Cu") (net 30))
 (segment (start 44.85 52.86) (end 44.853 52.857) (width 1.2) (layer "F.Cu") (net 10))
 (segment (start 44.853 52.857) (end 44.853 6.677) (width 1.2) (layer "F.Cu") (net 10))
 (segment (start 44.85 53.86) (end 44.85 52.86) (width 1.2) (layer "F.Cu") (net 10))
 (via (at 44.85 53.86) (size 1.2) (drill 0.6) (layers "F.Cu" "B.Cu") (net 10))
 (segment (start 44.85 53.86) (end 44.85 68.69) (width 1.2) (layer "B.Cu") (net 10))
 (segment (start 21.09 52.86) (end 21.093 52.857) (width 1.2) (layer "F.Cu") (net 4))
 (segment (start 21.09 53.86) (end 21.09 52.86) (width 1.2) (layer "F.Cu") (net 4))
 (segment (start 21.093 52.857) (end 21.093 6.677) (width 1.2) (layer "F.Cu") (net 4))
 (via (at 21.09 53.86) (size 1.2) (drill 0.6) (layers "F.Cu" "B.Cu") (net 4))
 (segment (start 21.09 53.86) (end 21.09 68.69) (width 1.2) (layer "B.Cu") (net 4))
 (segment (start 29.01 53.86) (end 29.01 52.86) (width 1.2) (layer "F.Cu") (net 6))
 (segment (start 29.01 52.86) (end 29.013 52.857) (width 1.2) (layer "F.Cu") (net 6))
 (segment (start 29.013 52.857) (end 29.013 6.677) (width 1.2) (layer "F.Cu") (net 6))
 (via (at 29.01 53.86) (size 1.2) (drill 0.6) (layers "F.Cu" "B.Cu") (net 6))
 (segment (start 29.01 53.86) (end 29.01 68.69) (width 1.2) (layer "B.Cu") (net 6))
 (segment (start 48.81 53.86) (end 48.81 68.69) (width 1.2) (layer "F.Cu") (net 33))
 (via (at 48.81 53.86) (size 1.2) (drill 0.6) (layers "F.Cu" "B.Cu") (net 33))
 (segment (start 48.81 53.86) (end 48.81 52.86) (width 1.2) (layer "B.Cu") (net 33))
 (segment (start 48.81 52.86) (end 48.813 52.857) (width 1.2) (layer "B.Cu") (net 33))
 (segment (start 48.813 52.857) (end 48.813 6.677) (width 1.2) (layer "B.Cu") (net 33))
 (segment (start 82.47 15.764) (end 80.493 13.787) (width 1.2) (layer "F.Cu") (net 17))
 (segment (start 74.55 53.86) (end 74.55 42.83) (width 1.2) (layer "F.Cu") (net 17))
 (segment (start 80.493 13.787) (end 80.493 6.677) (width 1.2) (layer "F.Cu") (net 17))
 (segment (start 74.55 42.83) (end 82.47 34.91) (width 1.2) (layer "F.Cu") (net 17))
 (segment (start 82.47 34.91) (end 82.47 15.764) (width 1.2) (layer "F.Cu") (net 17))
 (via (at 74.55 53.86) (size 1.2) (drill 0.6) (layers "F.Cu" "B.Cu") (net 17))
 (segment (start 72.57 60.84) (end 72.57 68.69) (width 1.2) (layer "B.Cu") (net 17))
 (segment (start 74.55 53.86) (end 74.55 58.86) (width 1.2) (layer "B.Cu") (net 17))
 (segment (start 74.55 58.86) (end 72.57 60.84) (width 1.2) (layer "B.Cu") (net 17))
 (segment (start 19.11 54.87) (end 17.13 56.85) (width 1.2) (layer "F.Cu") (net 25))
 (segment (start 17.13 56.85) (end 17.13 68.69) (width 1.2) (layer "F.Cu") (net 25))
 (segment (start 19.11 53.86) (end 19.11 54.87) (width 1.2) (layer "F.Cu") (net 25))
 (via (at 19.11 53.86) (size 1.2) (drill 0.6) (layers "F.Cu" "B.Cu") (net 25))
 (segment (start 19.1085 16.8485) (end 17.1315 14.8715) (width 1.2) (layer "B.Cu") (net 25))
 (segment (start 19.11 53.86) (end 19.11 52.86) (width 1.2) (layer "B.Cu") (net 25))
 (segment (start 17.1315 14.8715) (end 17.1315 6.6655) (width 1.2) (layer "B.Cu") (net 25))
 (segment (start 19.11 52.86) (end 19.1085 52.8585) (width 1.2) (layer "B.Cu") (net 25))
 (segment (start 19.1085 52.8585) (end 19.1085 16.8485) (width 1.2) (layer "B.Cu") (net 25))
 (segment (start 34.95 53.86) (end 34.95 54.87) (width 1.2) (layer "F.Cu") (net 29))
 (segment (start 34.95 54.87) (end 32.97 56.85) (width 1.2) (layer "F.Cu") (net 29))
 (segment (start 32.97 56.85) (end 32.97 68.69) (width 1.2) (layer "F.Cu") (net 29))
 (via (at 34.95 53.86) (size 1.2) (drill 0.6) (layers "F.Cu" "B.Cu") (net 29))
 (segment (start 34.95 53.86) (end 34.95 52.86) (width 1.2) (layer "B.Cu") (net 29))
 (segment (start 34.9485 16.8485) (end 32.9715 14.8715) (width 1.2) (layer "B.Cu") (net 29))
 (segment (start 32.9715 14.8715) (end 32.9715 6.6655) (width 1.2) (layer "B.Cu") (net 29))
 (segment (start 34.95 52.86) (end 34.9485 52.8585) (width 1.2) (layer "B.Cu") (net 29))
 (segment (start 34.9485 52.8585) (end 34.9485 16.8485) (width 1.2) (layer "B.Cu") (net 29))
 (segment (start 13.17 53.86) (end 13.17 52.86) (width 1.2) (layer "F.Cu") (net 2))
 (segment (start 13.17 52.86) (end 13.173 52.857) (width 1.2) (layer "F.Cu") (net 2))
 (segment (start 13.173 52.857) (end 13.173 6.677) (width 1.2) (layer "F.Cu") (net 2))
 (via (at 13.17 53.86) (size 1.2) (drill 0.6) (layers "F.Cu" "B.Cu") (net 2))
 (segment (start 13.17 53.86) (end 13.17 68.69) (width 1.2) (layer "B.Cu") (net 2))
 (segment (start 64.653 52.857) (end 64.653 6.677) (width 1.2) (layer "F.Cu") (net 15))
 (segment (start 64.65 53.86) (end 64.65 52.86) (width 1.2) (layer "F.Cu") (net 15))
 (segment (start 64.65 52.86) (end 64.653 52.857) (width 1.2) (layer "F.Cu") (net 15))
 (via (at 64.65 53.86) (size 1.2) (drill 0.6) (layers "F.Cu" "B.Cu") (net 15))
 (segment (start 64.65 53.86) (end 64.65 68.69) (width 1.2) (layer "B.Cu") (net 15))
 (segment (start 36.93 52.86) (end 36.933 52.857) (width 1.2) (layer "F.Cu") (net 8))
 (segment (start 36.93 53.86) (end 36.93 52.86) (width 1.2) (layer "F.Cu") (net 8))
 (segment (start 36.933 52.857) (end 36.933 6.677) (width 1.2) (layer "F.Cu") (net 8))
 (via (at 36.93 53.86) (size 1.2) (drill 0.6) (layers "F.Cu" "B.Cu") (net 8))
 (segment (start 36.93 53.86) (end 36.93 68.69) (width 1.2) (layer "B.Cu") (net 8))
 (segment (start 68.613 53.857) (end 68.613 6.677) (width 1.2) (layer "F.Cu") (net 16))
 (segment (start 68.61 53.86) (end 68.613 53.857) (width 1.2) (layer "F.Cu") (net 16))
 (via (at 68.61 53.86) (size 1.2) (drill 0.6) (layers "F.Cu" "B.Cu") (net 16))
 (segment (start 68.61 53.86) (end 68.61 68.69) (width 1.2) (layer "B.Cu") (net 16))
 (segment (start 32.973 52.857) (end 32.973 6.677) (width 1.2) (layer "F.Cu") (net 7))
 (segment (start 32.97 52.86) (end 32.973 52.857) (width 1.2) (layer "F.Cu") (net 7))
 (segment (start 32.97 53.86) (end 32.97 52.86) (width 1.2) (layer "F.Cu") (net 7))
 (via (at 32.97 53.86) (size 1.2) (drill 0.6) (layers "F.Cu" "B.Cu") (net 7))
 (segment (start 32.97 53.86) (end 32.97 68.69) (width 1.2) (layer "B.Cu") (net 7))
 (segment (start 23.07 54.875) (end 21.09 56.855) (width 1.2) (layer "F.Cu") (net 26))
 (segment (start 23.07 53.88) (end 23.07 54.875) (width 1.2) (layer "F.Cu") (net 26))
 (segment (start 21.09 56.855) (end 21.09 68.69) (width 1.2) (layer "F.Cu") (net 26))
 (via (at 23.07 53.88) (size 1.2) (drill 0.6) (layers "F.Cu" "B.Cu") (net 26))
 (segment (start 21.0915 14.8715) (end 21.0915 6.6655) (width 1.2) (layer "B.Cu") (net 26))
 (segment (start 23.07 53.88) (end 23.07 52.86) (width 1.2) (layer "B.Cu") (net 26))
 (segment (start 23.07 52.86) (end 23.0685 52.8585) (width 1.2) (layer "B.Cu") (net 26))
 (segment (start 23.0685 16.8485) (end 21.0915 14.8715) (width 1.2) (layer "B.Cu") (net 26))
 (segment (start 23.0685 52.8585) (end 23.0685 16.8485) (width 1.2) (layer "B.Cu") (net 26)))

